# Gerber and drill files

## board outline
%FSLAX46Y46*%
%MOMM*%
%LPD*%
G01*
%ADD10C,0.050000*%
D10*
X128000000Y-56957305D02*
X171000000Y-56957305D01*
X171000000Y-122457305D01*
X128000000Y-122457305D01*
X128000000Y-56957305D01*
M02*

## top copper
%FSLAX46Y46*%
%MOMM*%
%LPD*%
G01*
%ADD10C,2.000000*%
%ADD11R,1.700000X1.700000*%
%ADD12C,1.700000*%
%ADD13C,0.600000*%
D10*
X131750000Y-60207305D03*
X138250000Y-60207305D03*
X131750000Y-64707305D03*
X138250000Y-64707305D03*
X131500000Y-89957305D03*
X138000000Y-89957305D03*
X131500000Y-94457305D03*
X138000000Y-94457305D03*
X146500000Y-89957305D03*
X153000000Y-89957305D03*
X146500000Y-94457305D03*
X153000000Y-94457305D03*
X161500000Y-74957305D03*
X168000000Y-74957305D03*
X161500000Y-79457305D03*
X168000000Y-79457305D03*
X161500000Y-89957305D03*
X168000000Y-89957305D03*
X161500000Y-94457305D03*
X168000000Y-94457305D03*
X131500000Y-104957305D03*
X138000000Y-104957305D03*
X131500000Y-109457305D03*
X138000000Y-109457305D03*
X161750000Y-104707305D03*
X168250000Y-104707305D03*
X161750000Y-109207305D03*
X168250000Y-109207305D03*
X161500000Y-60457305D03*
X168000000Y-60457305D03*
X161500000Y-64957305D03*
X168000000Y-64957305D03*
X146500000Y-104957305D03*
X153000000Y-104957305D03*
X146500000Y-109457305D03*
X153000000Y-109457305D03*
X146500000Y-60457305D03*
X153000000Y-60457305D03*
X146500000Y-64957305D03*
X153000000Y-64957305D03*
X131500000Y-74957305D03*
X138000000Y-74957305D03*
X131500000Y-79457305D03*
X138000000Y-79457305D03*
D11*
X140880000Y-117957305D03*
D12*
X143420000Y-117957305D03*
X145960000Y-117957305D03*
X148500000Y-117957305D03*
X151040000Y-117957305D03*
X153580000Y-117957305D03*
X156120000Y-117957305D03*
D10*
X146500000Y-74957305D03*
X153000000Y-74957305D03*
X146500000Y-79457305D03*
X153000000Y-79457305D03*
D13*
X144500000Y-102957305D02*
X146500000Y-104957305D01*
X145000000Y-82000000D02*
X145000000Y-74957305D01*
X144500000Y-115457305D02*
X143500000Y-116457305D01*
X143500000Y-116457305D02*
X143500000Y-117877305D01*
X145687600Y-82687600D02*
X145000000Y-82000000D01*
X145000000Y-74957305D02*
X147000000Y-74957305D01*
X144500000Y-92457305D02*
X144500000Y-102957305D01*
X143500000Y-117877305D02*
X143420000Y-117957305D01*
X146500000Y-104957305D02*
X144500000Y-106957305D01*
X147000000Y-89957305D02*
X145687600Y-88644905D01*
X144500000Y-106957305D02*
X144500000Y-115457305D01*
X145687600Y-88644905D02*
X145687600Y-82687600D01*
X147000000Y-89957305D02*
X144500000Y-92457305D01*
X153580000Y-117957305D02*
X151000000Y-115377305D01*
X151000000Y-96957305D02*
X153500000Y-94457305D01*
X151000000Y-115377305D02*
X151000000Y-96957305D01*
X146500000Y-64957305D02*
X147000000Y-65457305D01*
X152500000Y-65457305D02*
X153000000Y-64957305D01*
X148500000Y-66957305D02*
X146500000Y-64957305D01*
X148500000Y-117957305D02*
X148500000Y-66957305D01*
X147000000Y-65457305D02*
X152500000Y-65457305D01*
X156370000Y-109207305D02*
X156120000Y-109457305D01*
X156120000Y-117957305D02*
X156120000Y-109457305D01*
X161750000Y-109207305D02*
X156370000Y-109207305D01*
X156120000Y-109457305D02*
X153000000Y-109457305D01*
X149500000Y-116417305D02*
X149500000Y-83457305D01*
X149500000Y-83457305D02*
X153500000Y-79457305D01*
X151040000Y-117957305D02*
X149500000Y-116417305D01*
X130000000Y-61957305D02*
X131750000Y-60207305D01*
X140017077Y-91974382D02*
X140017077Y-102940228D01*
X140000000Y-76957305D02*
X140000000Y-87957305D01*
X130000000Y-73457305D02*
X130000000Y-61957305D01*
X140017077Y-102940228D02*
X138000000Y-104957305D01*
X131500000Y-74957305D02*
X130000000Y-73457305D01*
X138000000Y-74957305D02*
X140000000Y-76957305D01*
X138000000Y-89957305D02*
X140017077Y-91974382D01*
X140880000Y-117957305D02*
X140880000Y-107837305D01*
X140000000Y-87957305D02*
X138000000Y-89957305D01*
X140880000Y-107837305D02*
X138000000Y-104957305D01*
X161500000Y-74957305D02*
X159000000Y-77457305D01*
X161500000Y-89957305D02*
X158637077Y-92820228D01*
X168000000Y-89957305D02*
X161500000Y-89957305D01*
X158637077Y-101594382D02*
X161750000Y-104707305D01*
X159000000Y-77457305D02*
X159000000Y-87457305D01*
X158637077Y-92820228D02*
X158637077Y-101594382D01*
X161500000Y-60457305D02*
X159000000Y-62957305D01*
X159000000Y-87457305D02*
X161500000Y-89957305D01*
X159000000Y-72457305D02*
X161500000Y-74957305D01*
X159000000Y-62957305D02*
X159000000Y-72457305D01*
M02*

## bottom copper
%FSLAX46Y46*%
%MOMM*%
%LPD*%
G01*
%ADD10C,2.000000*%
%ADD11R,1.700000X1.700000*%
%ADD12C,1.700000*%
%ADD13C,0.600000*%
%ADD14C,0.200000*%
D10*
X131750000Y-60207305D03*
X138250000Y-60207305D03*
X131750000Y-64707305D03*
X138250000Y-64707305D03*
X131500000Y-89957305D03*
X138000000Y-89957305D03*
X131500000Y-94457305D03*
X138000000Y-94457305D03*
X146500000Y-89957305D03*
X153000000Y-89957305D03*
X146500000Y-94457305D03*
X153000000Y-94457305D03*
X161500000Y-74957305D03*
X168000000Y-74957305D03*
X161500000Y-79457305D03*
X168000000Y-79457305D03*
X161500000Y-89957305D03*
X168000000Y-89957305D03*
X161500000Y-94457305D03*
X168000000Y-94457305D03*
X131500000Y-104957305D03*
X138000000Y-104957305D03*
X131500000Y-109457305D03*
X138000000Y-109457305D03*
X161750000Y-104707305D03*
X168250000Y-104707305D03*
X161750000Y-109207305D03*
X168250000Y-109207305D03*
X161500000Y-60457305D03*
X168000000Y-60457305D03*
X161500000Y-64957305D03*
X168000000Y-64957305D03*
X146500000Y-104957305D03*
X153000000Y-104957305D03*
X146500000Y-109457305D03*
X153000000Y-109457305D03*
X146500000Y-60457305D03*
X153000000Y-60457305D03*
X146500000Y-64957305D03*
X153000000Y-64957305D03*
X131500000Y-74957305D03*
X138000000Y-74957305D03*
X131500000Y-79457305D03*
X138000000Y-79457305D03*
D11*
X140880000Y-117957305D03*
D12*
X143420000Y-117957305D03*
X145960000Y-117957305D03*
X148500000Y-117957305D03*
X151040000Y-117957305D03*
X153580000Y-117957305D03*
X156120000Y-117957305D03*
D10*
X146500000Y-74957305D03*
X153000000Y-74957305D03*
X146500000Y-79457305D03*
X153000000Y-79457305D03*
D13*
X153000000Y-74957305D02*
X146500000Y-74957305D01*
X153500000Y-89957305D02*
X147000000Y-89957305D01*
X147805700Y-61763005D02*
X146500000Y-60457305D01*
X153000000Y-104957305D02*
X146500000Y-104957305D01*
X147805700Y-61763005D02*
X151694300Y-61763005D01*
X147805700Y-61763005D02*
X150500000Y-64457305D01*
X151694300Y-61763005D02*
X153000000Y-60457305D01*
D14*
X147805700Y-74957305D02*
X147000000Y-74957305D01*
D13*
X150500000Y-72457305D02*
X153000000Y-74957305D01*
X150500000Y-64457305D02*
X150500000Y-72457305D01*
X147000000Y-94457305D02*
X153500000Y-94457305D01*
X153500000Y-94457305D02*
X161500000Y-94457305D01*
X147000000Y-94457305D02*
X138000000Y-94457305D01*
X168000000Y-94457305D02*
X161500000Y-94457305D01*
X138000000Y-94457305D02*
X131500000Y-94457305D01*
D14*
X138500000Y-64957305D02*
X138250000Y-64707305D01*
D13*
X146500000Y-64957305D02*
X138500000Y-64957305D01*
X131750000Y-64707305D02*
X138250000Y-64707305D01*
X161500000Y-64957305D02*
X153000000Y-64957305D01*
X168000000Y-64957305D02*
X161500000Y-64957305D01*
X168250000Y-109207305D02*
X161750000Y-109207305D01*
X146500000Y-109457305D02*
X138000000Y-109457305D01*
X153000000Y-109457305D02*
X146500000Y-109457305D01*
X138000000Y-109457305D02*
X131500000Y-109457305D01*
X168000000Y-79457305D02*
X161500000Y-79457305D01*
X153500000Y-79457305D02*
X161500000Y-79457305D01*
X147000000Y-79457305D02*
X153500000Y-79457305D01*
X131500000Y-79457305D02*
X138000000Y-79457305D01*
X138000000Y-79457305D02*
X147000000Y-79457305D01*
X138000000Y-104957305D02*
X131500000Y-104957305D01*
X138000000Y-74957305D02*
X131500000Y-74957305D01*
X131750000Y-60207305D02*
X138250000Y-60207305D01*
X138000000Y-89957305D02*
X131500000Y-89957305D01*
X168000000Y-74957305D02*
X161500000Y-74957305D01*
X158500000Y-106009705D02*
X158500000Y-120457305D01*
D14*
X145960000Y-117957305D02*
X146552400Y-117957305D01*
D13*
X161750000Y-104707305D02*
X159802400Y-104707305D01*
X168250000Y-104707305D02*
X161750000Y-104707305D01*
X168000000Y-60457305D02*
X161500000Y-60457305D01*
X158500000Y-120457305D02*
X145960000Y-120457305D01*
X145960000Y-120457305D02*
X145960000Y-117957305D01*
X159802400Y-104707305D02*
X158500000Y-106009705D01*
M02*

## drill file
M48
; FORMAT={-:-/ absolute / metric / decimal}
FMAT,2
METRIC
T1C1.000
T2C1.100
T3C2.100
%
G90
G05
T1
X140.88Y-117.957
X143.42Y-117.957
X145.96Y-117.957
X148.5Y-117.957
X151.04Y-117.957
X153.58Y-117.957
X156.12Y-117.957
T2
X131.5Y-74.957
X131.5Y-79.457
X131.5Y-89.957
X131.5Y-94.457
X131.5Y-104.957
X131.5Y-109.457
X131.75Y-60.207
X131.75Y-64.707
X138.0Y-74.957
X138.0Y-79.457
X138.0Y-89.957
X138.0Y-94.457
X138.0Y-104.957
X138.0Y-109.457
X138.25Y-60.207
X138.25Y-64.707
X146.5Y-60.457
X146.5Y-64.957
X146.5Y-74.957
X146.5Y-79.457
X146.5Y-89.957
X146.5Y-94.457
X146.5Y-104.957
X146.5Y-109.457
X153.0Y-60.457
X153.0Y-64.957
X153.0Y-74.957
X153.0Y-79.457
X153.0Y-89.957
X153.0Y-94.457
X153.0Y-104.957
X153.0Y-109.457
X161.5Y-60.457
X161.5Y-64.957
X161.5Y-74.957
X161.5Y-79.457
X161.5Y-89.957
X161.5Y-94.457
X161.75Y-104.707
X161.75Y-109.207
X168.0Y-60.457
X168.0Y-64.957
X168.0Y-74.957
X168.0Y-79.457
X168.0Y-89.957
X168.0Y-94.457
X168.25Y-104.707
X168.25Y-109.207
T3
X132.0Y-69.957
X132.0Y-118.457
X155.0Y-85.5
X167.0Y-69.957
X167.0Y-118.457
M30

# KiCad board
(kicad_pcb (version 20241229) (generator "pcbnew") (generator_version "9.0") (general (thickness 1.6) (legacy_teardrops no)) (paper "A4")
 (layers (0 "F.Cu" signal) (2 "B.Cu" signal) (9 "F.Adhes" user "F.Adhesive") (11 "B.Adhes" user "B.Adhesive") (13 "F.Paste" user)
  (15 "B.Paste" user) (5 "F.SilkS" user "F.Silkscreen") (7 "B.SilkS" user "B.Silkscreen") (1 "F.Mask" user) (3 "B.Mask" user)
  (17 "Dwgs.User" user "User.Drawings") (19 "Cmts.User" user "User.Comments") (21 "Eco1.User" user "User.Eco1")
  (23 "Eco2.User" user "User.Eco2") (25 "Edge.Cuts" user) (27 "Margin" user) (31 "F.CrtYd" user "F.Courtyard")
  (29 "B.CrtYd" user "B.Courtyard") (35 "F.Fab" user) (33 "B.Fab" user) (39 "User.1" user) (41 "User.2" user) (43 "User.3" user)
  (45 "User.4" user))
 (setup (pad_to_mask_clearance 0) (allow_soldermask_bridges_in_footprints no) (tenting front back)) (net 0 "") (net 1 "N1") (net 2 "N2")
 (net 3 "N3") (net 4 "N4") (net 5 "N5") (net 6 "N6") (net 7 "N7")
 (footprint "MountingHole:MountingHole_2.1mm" (layer "F.Cu") (at 167 69.957305)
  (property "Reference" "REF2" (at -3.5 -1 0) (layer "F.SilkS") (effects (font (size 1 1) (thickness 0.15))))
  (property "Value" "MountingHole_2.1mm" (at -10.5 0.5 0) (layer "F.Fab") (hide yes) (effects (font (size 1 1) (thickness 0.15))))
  (pad "" np_thru_hole circle (at 0 0) (size 2.1 2.1) (drill 2.1) (layers "*.Cu" "*.Mask")))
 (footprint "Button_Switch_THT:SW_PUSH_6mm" (layer "F.Cu") (at 131.75 60.207305)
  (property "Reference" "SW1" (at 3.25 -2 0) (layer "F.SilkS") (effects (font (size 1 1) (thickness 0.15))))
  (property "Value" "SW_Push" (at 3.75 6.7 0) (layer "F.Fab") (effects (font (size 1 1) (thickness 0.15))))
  (pad "1" thru_hole circle (at 0 0 90) (size 2 2) (drill 1.1) (layers "*.Cu" "*.Mask") (remove_unused_layers no) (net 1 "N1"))
  (pad "1" thru_hole circle (at 6.5 0 90) (size 2 2) (drill 1.1) (layers "*.Cu" "*.Mask") (remove_unused_layers no) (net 1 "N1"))
  (pad "2" thru_hole circle (at 0 4.5 90) (size 2 2) (drill 1.1) (layers "*.Cu" "*.Mask") (remove_unused_layers no) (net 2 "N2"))
  (pad "2" thru_hole circle (at 6.5 4.5 90) (size 2 2) (drill 1.1) (layers "*.Cu" "*.Mask") (remove_unused_layers no) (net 2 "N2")))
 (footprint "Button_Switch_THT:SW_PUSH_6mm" (layer "F.Cu") (at 131.5 89.957305)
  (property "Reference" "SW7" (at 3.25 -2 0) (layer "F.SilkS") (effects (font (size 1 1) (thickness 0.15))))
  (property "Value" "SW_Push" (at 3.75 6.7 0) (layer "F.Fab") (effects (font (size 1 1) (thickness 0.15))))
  (pad "1" thru_hole circle (at 0 0 90) (size 2 2) (drill 1.1) (layers "*.Cu" "*.Mask") (remove_unused_layers no) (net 1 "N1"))
  (pad "1" thru_hole circle (at 6.5 0 90) (size 2 2) (drill 1.1) (layers "*.Cu" "*.Mask") (remove_unused_layers no) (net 1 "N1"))
  (pad "2" thru_hole circle (at 0 4.5 90) (size 2 2) (drill 1.1) (layers "*.Cu" "*.Mask") (remove_unused_layers no) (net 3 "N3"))
  (pad "2" thru_hole circle (at 6.5 4.5 90) (size 2 2) (drill 1.1) (layers "*.Cu" "*.Mask") (remove_unused_layers no) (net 3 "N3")))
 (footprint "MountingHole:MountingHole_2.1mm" (layer "F.Cu") (at 132 69.957305)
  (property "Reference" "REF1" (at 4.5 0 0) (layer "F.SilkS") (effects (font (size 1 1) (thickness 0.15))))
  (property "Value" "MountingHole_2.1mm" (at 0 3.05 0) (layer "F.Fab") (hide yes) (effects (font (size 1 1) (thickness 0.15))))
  (pad "" np_thru_hole circle (at 0 0) (size 2.1 2.1) (drill 2.1) (layers "*.Cu" "*.Mask")))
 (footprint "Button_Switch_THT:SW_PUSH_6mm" (layer "F.Cu") (at 146.5 89.957305)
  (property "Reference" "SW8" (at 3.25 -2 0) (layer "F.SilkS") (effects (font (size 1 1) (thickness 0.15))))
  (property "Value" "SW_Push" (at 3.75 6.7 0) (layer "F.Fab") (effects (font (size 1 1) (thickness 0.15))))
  (pad "1" thru_hole circle (at 0 0 90) (size 2 2) (drill 1.1) (layers "*.Cu" "*.Mask") (remove_unused_layers no) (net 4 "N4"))
  (pad "1" thru_hole circle (at 6.5 0 90) (size 2 2) (drill 1.1) (layers "*.Cu" "*.Mask") (remove_unused_layers no) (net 4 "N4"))
  (pad "2" thru_hole circle (at 0 4.5 90) (size 2 2) (drill 1.1) (layers "*.Cu" "*.Mask") (remove_unused_layers no) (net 3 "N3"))
  (pad "2" thru_hole circle (at 6.5 4.5 90) (size 2 2) (drill 1.1) (layers "*.Cu" "*.Mask") (remove_unused_layers no) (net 3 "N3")))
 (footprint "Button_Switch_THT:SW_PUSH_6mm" (layer "F.Cu") (at 161.5 74.957305)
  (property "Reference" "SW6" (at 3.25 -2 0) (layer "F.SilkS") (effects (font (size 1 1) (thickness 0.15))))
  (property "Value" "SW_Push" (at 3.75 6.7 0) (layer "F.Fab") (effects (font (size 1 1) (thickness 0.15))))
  (pad "1" thru_hole circle (at 0 0 90) (size 2 2) (drill 1.1) (layers "*.Cu" "*.Mask") (remove_unused_layers no) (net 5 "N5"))
  (pad "1" thru_hole circle (at 6.5 0 90) (size 2 2) (drill 1.1) (layers "*.Cu" "*.Mask") (remove_unused_layers no) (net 5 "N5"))
  (pad "2" thru_hole circle (at 0 4.5 90) (size 2 2) (drill 1.1) (layers "*.Cu" "*.Mask") (remove_unused_layers no) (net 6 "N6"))
  (pad "2" thru_hole circle (at 6.5 4.5 90) (size 2 2) (drill 1.1) (layers "*.Cu" "*.Mask") (remove_unused_layers no) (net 6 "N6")))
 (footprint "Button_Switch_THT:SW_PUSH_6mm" (layer "F.Cu") (at 161.5 89.957305)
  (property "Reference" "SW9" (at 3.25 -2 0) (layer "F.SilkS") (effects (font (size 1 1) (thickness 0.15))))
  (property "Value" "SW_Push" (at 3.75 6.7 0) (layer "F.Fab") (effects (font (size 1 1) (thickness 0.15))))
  (pad "1" thru_hole circle (at 0 0 90) (size 2 2) (drill 1.1) (layers "*.Cu" "*.Mask") (remove_unused_layers no) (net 5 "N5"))
  (pad "1" thru_hole circle (at 6.5 0 90) (size 2 2) (drill 1.1) (layers "*.Cu" "*.Mask") (remove_unused_layers no) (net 5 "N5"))
  (pad "2" thru_hole circle (at 0 4.5 90) (size 2 2) (drill 1.1) (layers "*.Cu" "*.Mask") (remove_unused_layers no) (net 3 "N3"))
  (pad "2" thru_hole circle (at 6.5 4.5 90) (size 2 2) (drill 1.1) (layers "*.Cu" "*.Mask") (remove_unused_layers no) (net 3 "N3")))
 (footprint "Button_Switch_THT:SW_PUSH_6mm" (layer "F.Cu") (at 131.5 104.957305)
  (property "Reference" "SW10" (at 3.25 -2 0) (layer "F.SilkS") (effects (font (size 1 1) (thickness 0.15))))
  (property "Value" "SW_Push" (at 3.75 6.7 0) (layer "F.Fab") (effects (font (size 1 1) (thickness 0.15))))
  (pad "1" thru_hole circle (at 0 0 90) (size 2 2) (drill 1.1) (layers "*.Cu" "*.Mask") (remove_unused_layers no) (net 1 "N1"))
  (pad "1" thru_hole circle (at 6.5 0 90) (size 2 2) (drill 1.1) (layers "*.Cu" "*.Mask") (remove_unused_layers no) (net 1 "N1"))
  (pad "2" thru_hole circle (at 0 4.5 90) (size 2 2) (drill 1.1) (layers "*.Cu" "*.Mask") (remove_unused_layers no) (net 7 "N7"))
  (pad "2" thru_hole circle (at 6.5 4.5 90) (size 2 2) (drill 1.1) (layers "*.Cu" "*.Mask") (remove_unused_layers no) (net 7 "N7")))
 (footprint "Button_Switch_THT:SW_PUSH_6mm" (layer "F.Cu") (at 161.75 104.707305)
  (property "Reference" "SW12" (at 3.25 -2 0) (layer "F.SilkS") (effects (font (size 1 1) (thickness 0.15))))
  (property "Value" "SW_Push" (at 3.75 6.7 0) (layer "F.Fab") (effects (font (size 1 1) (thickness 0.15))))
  (pad "1" thru_hole circle (at 0 0 90) (size 2 2) (drill 1.1) (layers "*.Cu" "*.Mask") (remove_unused_layers no) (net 5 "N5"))
  (pad "1" thru_hole circle (at 6.5 0 90) (size 2 2) (drill 1.1) (layers "*.Cu" "*.Mask") (remove_unused_layers no) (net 5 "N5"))
  (pad "2" thru_hole circle (at 0 4.5 90) (size 2 2) (drill 1.1) (layers "*.Cu" "*.Mask") (remove_unused_layers no) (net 7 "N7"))
  (pad "2" thru_hole circle (at 6.5 4.5 90) (size 2 2) (drill 1.1) (layers "*.Cu" "*.Mask") (remove_unused_layers no) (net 7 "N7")))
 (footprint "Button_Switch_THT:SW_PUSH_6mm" (layer "F.Cu") (at 161.5 60.457305)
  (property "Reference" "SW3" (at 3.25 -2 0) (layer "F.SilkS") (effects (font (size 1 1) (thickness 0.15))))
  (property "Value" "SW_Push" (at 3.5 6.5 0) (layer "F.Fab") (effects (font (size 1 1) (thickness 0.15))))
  (pad "1" thru_hole circle (at 0 0 90) (size 2 2) (drill 1.1) (layers "*.Cu" "*.Mask") (remove_unused_layers no) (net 5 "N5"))
  (pad "1" thru_hole circle (at 6.5 0 90) (size 2 2) (drill 1.1) (layers "*.Cu" "*.Mask") (remove_unused_layers no) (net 5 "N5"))
  (pad "2" thru_hole circle (at 0 4.5 90) (size 2 2) (drill 1.1) (layers "*.Cu" "*.Mask") (remove_unused_layers no) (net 2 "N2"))
  (pad "2" thru_hole circle (at 6.5 4.5 90) (size 2 2) (drill 1.1) (layers "*.Cu" "*.Mask") (remove_unused_layers no) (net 2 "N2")))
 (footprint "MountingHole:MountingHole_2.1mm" (layer "F.Cu") (at 155 85.5)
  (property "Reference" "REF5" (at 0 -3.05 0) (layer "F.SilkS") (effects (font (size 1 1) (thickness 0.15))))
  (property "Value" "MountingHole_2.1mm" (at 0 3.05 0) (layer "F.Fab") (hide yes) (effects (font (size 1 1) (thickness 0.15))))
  (pad "" np_thru_hole circle (at 0 0) (size 2.1 2.1) (drill 2.1) (layers "*.Cu" "*.Mask")))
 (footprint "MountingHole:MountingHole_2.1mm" (layer "F.Cu") (at 132 118.457305)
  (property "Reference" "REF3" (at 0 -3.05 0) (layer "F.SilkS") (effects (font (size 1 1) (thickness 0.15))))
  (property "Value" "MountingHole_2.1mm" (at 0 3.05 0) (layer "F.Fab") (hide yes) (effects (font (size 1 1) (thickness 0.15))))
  (pad "" np_thru_hole circle (at 0 0) (size 2.1 2.1) (drill 2.1) (layers "*.Cu" "*.Mask")))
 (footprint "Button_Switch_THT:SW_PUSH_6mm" (layer "F.Cu") (at 146.5 104.957305)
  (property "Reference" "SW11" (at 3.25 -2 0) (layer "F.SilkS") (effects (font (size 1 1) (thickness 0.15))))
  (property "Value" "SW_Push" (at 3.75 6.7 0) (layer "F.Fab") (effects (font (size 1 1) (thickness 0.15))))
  (pad "1" thru_hole circle (at 0 0 90) (size 2 2) (drill 1.1) (layers "*.Cu" "*.Mask") (remove_unused_layers no) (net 4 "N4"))
  (pad "1" thru_hole circle (at 6.5 0 90) (size 2 2) (drill 1.1) (layers "*.Cu" "*.Mask") (remove_unused_layers no) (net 4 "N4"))
  (pad "2" thru_hole circle (at 0 4.5 90) (size 2 2) (drill 1.1) (layers "*.Cu" "*.Mask") (remove_unused_layers no) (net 7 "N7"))
  (pad "2" thru_hole circle (at 6.5 4.5 90) (size 2 2) (drill 1.1) (layers "*.Cu" "*.Mask") (remove_unused_layers no) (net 7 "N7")))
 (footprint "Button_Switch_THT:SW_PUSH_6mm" (layer "F.Cu") (at 146.5 60.457305)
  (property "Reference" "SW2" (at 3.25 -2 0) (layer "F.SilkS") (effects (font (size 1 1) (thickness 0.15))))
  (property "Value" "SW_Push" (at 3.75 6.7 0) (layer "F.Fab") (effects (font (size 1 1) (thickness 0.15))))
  (pad "1" thru_hole circle (at 0 0 90) (size 2 2) (drill 1.1) (layers "*.Cu" "*.Mask") (remove_unused_layers no) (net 4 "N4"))
  (pad "1" thru_hole circle (at 6.5 0 90) (size 2 2) (drill 1.1) (layers "*.Cu" "*.Mask") (remove_unused_layers no) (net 4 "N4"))
  (pad "2" thru_hole circle (at 0 4.5 90) (size 2 2) (drill 1.1) (layers "*.Cu" "*.Mask") (remove_unused_layers no) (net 2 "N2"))
  (pad "2" thru_hole circle (at 6.5 4.5 90) (size 2 2) (drill 1.1) (layers "*.Cu" "*.Mask") (remove_unused_layers no) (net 2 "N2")))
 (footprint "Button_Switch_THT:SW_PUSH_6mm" (layer "F.Cu") (at 131.5 74.957305)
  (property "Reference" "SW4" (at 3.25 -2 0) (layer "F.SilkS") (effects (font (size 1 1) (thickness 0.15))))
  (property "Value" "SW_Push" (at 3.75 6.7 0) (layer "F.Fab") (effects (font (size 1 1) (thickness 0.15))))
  (pad "1" thru_hole circle (at 0 0 90) (size 2 2) (drill 1.1) (layers "*.Cu" "*.Mask") (remove_unused_layers no) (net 1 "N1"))
  (pad "1" thru_hole circle (at 6.5 0 90) (size 2 2) (drill 1.1) (layers "*.Cu" "*.Mask") (remove_unused_layers no) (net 1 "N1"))
  (pad "2" thru_hole circle (at 0 4.5 90) (size 2 2) (drill 1.1) (layers "*.Cu" "*.Mask") (remove_unused_layers no) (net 6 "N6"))
  (pad "2" thru_hole circle (at 6.5 4.5 90) (size 2 2) (drill 1.1) (layers "*.Cu" "*.Mask") (remove_unused_layers no) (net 6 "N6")))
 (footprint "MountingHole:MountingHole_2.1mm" (layer "F.Cu") (at 167 118.457305)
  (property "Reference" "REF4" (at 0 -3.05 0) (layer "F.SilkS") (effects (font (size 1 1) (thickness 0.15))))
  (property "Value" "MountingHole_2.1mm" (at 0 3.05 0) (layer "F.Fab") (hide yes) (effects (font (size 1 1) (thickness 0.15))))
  (pad "" np_thru_hole circle (at 0 0) (size 2.1 2.1) (drill 2.1) (layers "*.Cu" "*.Mask")))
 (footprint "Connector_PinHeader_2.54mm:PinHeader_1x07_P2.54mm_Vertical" (layer "F.Cu") (at 140.88 117.957305 90)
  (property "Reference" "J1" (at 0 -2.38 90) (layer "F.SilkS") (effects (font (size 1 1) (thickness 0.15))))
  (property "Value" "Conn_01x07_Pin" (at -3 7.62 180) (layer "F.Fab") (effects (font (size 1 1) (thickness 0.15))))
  (pad "1" thru_hole rect (at 0 0 90) (size 1.7 1.7) (drill 1) (layers "*.Cu" "*.Mask") (remove_unused_layers no) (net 1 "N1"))
  (pad "2" thru_hole circle (at 0 2.54 90) (size 1.7 1.7) (drill 1) (layers "*.Cu" "*.Mask") (remove_unused_layers no) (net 4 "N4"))
  (pad "3" thru_hole circle (at 0 5.08 90) (size 1.7 1.7) (drill 1) (layers "*.Cu" "*.Mask") (remove_unused_layers no) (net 5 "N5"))
  (pad "4" thru_hole circle (at 0 7.62 90) (size 1.7 1.7) (drill 1) (layers "*.Cu" "*.Mask") (remove_unused_layers no) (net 2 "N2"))
  (pad "5" thru_hole circle (at 0 10.16 90) (size 1.7 1.7) (drill 1) (layers "*.Cu" "*.Mask") (remove_unused_layers no) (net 6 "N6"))
  (pad "6" thru_hole circle (at 0 12.7 90) (size 1.7 1.7) (drill 1) (layers "*.Cu" "*.Mask") (remove_unused_layers no) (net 3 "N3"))
  (pad "7" thru_hole circle (at 0 15.24 90) (size 1.7 1.7) (drill 1) (layers "*.Cu" "*.Mask") (remove_unused_layers no) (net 7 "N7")))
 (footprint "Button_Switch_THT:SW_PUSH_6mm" (layer "F.Cu") (at 146.5 74.957305)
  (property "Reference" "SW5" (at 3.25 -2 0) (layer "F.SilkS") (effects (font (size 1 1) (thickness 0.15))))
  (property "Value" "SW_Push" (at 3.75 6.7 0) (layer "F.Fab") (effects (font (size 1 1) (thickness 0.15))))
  (pad "1" thru_hole circle (at 0 0 90) (size 2 2) (drill 1.1) (layers "*.Cu" "*.Mask") (remove_unused_layers no) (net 4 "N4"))
  (pad "1" thru_hole circle (at 6.5 0 90) (size 2 2) (drill 1.1) (layers "*.Cu" "*.Mask") (remove_unused_layers no) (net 4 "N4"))
  (pad "2" thru_hole circle (at 0 4.5 90) (size 2 2) (drill 1.1) (layers "*.Cu" "*.Mask") (remove_unused_layers no) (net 6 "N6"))
  (pad "2" thru_hole circle (at 6.5 4.5 90) (size 2 2) (drill 1.1) (layers "*.Cu" "*.Mask") (remove_unused_layers no) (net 6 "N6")))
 (gr_rect (start 128 56.957305) (end 171 122.457305) (stroke (width 0.05) (type default)) (fill no) (layer "Edge.Cuts"))
 (segment (start 144.5 102.957305) (end 146.5 104.957305) (width 0.6) (layer "F.Cu") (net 4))
 (segment (start 145 82) (end 145 74.957305) (width 0.6) (layer "F.Cu") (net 4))
 (segment (start 144.5 115.457305) (end 143.5 116.457305) (width 0.6) (layer "F.Cu") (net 4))
 (segment (start 143.5 116.457305) (end 143.5 117.877305) (width 0.6) (layer "F.Cu") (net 4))
 (segment (start 145.6876 82.6876) (end 145 82) (width 0.6) (layer "F.Cu") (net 4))
 (segment (start 145 74.957305) (end 147 74.957305) (width 0.6) (layer "F.Cu") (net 4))
 (segment (start 144.5 92.457305) (end 144.5 102.957305) (width 0.6) (layer "F.Cu") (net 4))
 (segment (start 143.5 117.877305) (end 143.42 117.957305) (width 0.6) (layer "F.Cu") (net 4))
 (segment (start 146.5 104.957305) (end 144.5 106.957305) (width 0.6) (layer "F.Cu") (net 4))
 (segment (start 147 89.957305) (end 145.6876 88.644905) (width 0.6) (layer "F.Cu") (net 4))
 (segment (start 144.5 106.957305) (end 144.5 115.457305) (width 0.6) (layer "F.Cu") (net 4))
 (segment (start 145.6876 88.644905) (end 145.6876 82.6876) (width 0.6) (layer "F.Cu") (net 4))
 (segment (start 147 89.957305) (end 144.5 92.457305) (width 0.6) (layer "F.Cu") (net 4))
 (segment (start 153 74.957305) (end 146.5 74.957305) (width 0.6) (layer "B.Cu") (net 4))
 (segment (start 153.5 89.957305) (end 147 89.957305) (width 0.6) (layer "B.Cu") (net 4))
 (segment (start 147.8057 61.763005) (end 146.5 60.457305) (width 0.6) (layer "B.Cu") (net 4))
 (segment (start 153 104.957305) (end 146.5 104.957305) (width 0.6) (layer "B.Cu") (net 4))
 (segment (start 147.8057 61.763005) (end 151.6943 61.763005) (width 0.6) (layer "B.Cu") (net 4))
 (segment (start 147.8057 61.763005) (end 150.5 64.457305) (width 0.6) (layer "B.Cu") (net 4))
 (segment (start 151.6943 61.763005) (end 153 60.457305) (width 0.6) (layer "B.Cu") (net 4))
 (segment (start 147.8057 74.957305) (end 147 74.957305) (width 0.2) (layer "B.Cu") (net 4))
 (segment (start 150.5 72.457305) (end 153 74.957305) (width 0.6) (layer "B.Cu") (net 4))
 (segment (start 150.5 64.457305) (end 150.5 72.457305) (width 0.6) (layer "B.Cu") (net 4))
 (segment (start 153.58 117.957305) (end 151 115.377305) (width 0.6) (layer "F.Cu") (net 3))
 (segment (start 151 96.957305) (end 153.5 94.457305) (width 0.6) (layer "F.Cu") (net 3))
 (segment (start 151 115.377305) (end 151 96.957305) (width 0.6) (layer "F.Cu") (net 3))
 (segment (start 147 94.457305) (end 153.5 94.457305) (width 0.6) (layer "B.Cu") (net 3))
 (segment (start 153.5 94.457305) (end 161.5 94.457305) (width 0.6) (layer "B.Cu") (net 3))
 (segment (start 147 94.457305) (end 138 94.457305) (width 0.6) (layer "B.Cu") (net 3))
 (segment (start 168 94.457305) (end 161.5 94.457305) (width 0.6) (layer "B.Cu") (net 3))
 (segment (start 138 94.457305) (end 131.5 94.457305) (width 0.6) (layer "B.Cu") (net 3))
 (segment (start 146.5 64.957305) (end 147 65.457305) (width 0.6) (layer "F.Cu") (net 2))
 (segment (start 152.5 65.457305) (end 153 64.957305) (width 0.6) (layer "F.Cu") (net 2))
 (segment (start 148.5 66.957305) (end 146.5 64.957305) (width 0.6) (layer "F.Cu") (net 2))
 (segment (start 148.5 117.957305) (end 148.5 66.957305) (width 0.6) (layer "F.Cu") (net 2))
 (segment (start 147 65.457305) (end 152.5 65.457305) (width 0.6) (layer "F.Cu") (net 2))
 (segment (start 138.5 64.957305) (end 138.25 64.707305) (width 0.2) (layer "B.Cu") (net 2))
 (segment (start 146.5 64.957305) (end 138.5 64.957305) (width 0.6) (layer "B.Cu") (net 2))
 (segment (start 131.75 64.707305) (end 138.25 64.707305) (width 0.6) (layer "B.Cu") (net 2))
 (segment (start 161.5 64.957305) (end 153 64.957305) (width 0.6) (layer "B.Cu") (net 2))
 (segment (start 168 64.957305) (end 161.5 64.957305) (width 0.6) (layer "B.Cu") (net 2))
 (segment (start 156.37 109.207305) (end 156.12 109.457305) (width 0.6) (layer "F.Cu") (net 7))
 (segment (start 156.12 117.957305) (end 156.12 109.457305) (width 0.6) (layer "F.Cu") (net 7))
 (segment (start 161.75 109.207305) (end 156.37 109.207305) (width 0.6) (layer "F.Cu") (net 7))
 (segment (start 156.12 109.457305) (end 153 109.457305) (width 0.6) (layer "F.Cu") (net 7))
 (segment (start 168.25 109.207305) (end 161.75 109.207305) (width 0.6) (layer "B.Cu") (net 7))
 (segment (start 146.5 109.457305) (end 138 109.457305) (width 0.6) (layer "B.Cu") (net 7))
 (segment (start 153 109.457305) (end 146.5 109.457305) (width 0.6) (layer "B.Cu") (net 7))
 (segment (start 138 109.457305) (end 131.5 109.457305) (width 0.6) (layer "B.Cu") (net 7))
 (segment (start 149.5 116.417305) (end 149.5 83.457305) (width 0.6) (layer "F.Cu") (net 6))
 (segment (start 149.5 83.457305) (end 153.5 79.457305) (width 0.6) (layer "F.Cu") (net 6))
 (segment (start 151.04 117.957305) (end 149.5 116.417305) (width 0.6) (layer "F.Cu") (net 6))
 (segment (start 168 79.457305) (end 161.5 79.457305) (width 0.6) (layer "B.Cu") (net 6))
 (segment (start 153.5 79.457305) (end 161.5 79.457305) (width 0.6) (layer "B.Cu") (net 6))
 (segment (start 147 79.457305) (end 153.5 79.457305) (width 0.6) (layer "B.Cu") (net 6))
 (segment (start 131.5 79.457305) (end 138 79.457305) (width 0.6) (layer "B.Cu") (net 6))
 (segment (start 138 79.457305) (end 147 79.457305) (width 0.6) (layer "B.Cu") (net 6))
 (segment (start 130 61.957305) (end 131.75 60.207305) (width 0.6) (layer "F.Cu") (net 1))
 (segment (start 140.017077 91.974382) (end 140.017077 102.940228) (width 0.6) (layer "F.Cu") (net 1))
 (segment (start 140 76.957305) (end 140 87.957305) (width 0.6) (layer "F.Cu") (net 1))
 (segment (start 130 73.457305) (end 130 61.957305) (width 0.6) (layer "F.Cu") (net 1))
 (segment (start 140.017077 102.940228) (end 138 104.957305) (width 0.6) (layer "F.Cu") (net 1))
 (segment (start 131.5 74.957305) (end 130 73.457305) (width 0.6) (layer "F.Cu") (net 1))
 (segment (start 138 74.957305) (end 140 76.957305) (width 0.6) (layer "F.Cu") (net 1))
 (segment (start 138 89.957305) (end 140.017077 91.974382) (width 0.6) (layer "F.Cu") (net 1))
 (segment (start 140.88 117.957305) (end 140.88 107.837305) (width 0.6) (layer "F.Cu") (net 1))
 (segment (start 140 87.957305) (end 138 89.957305) (width 0.6) (layer "F.Cu") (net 1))
 (segment (start 140.88 107.837305) (end 138 104.957305) (width 0.6) (layer "F.Cu") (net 1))
 (segment (start 138 104.957305) (end 131.5 104.957305) (width 0.6) (layer "B.Cu") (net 1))
 (segment (start 138 74.957305) (end 131.5 74.957305) (width 0.6) (layer "B.Cu") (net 1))
 (segment (start 131.75 60.207305) (end 138.25 60.207305) (width 0.6) (layer "B.Cu") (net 1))
 (segment (start 138 89.957305) (end 131.5 89.957305) (width 0.6) (layer "B.Cu") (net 1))
 (segment (start 161.5 74.957305) (end 159 77.457305) (width 0.6) (layer "F.Cu") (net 5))
 (segment (start 161.5 89.957305) (end 158.637077 92.820228) (width 0.6) (layer "F.Cu") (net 5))
 (segment (start 168 89.957305) (end 161.5 89.957305) (width 0.6) (layer "F.Cu") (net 5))
 (segment (start 158.637077 101.594382) (end 161.75 104.707305) (width 0.6) (layer "F.Cu") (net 5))
 (segment (start 159 77.457305) (end 159 87.457305) (width 0.6) (layer "F.Cu") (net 5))
 (segment (start 158.637077 92.820228) (end 158.637077 101.594382) (width 0.6) (layer "F.Cu") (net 5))
 (segment (start 161.5 60.457305) (end 159 62.957305) (width 0.6) (layer "F.Cu") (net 5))
 (segment (start 159 87.457305) (end 161.5 89.957305) (width 0.6) (layer "F.Cu") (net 5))
 (segment (start 159 72.457305) (end 161.5 74.957305) (width 0.6) (layer "F.Cu") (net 5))
 (segment (start 159 62.957305) (end 159 72.457305) (width 0.6) (layer "F.Cu") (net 5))
 (segment (start 168 74.957305) (end 161.5 74.957305) (width 0.6) (layer "B.Cu") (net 5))
 (segment (start 158.5 106.009705) (end 158.5 120.457305) (width 0.6) (layer "B.Cu") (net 5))
 (segment (start 145.96 117.957305) (end 146.5524 117.957305) (width 0.2) (layer "B.Cu") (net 5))
 (segment (start 161.75 104.707305) (end 159.8024 104.707305) (width 0.6) (layer "B.Cu") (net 5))
 (segment (start 168.25 104.707305) (end 161.75 104.707305) (width 0.6) (layer "B.Cu") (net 5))
 (segment (start 168 60.457305) (end 161.5 60.457305) (width 0.6) (layer "B.Cu") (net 5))
 (segment (start 158.5 120.457305) (end 145.96 120.457305) (width 0.6) (layer "B.Cu") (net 5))
 (segment (start 145.96 120.457305) (end 145.96 117.957305) (width 0.6) (layer "B.Cu") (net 5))
 (segment (start 159.8024 104.707305) (end 158.5 106.009705) (width 0.6) (layer "B.Cu") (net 5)))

